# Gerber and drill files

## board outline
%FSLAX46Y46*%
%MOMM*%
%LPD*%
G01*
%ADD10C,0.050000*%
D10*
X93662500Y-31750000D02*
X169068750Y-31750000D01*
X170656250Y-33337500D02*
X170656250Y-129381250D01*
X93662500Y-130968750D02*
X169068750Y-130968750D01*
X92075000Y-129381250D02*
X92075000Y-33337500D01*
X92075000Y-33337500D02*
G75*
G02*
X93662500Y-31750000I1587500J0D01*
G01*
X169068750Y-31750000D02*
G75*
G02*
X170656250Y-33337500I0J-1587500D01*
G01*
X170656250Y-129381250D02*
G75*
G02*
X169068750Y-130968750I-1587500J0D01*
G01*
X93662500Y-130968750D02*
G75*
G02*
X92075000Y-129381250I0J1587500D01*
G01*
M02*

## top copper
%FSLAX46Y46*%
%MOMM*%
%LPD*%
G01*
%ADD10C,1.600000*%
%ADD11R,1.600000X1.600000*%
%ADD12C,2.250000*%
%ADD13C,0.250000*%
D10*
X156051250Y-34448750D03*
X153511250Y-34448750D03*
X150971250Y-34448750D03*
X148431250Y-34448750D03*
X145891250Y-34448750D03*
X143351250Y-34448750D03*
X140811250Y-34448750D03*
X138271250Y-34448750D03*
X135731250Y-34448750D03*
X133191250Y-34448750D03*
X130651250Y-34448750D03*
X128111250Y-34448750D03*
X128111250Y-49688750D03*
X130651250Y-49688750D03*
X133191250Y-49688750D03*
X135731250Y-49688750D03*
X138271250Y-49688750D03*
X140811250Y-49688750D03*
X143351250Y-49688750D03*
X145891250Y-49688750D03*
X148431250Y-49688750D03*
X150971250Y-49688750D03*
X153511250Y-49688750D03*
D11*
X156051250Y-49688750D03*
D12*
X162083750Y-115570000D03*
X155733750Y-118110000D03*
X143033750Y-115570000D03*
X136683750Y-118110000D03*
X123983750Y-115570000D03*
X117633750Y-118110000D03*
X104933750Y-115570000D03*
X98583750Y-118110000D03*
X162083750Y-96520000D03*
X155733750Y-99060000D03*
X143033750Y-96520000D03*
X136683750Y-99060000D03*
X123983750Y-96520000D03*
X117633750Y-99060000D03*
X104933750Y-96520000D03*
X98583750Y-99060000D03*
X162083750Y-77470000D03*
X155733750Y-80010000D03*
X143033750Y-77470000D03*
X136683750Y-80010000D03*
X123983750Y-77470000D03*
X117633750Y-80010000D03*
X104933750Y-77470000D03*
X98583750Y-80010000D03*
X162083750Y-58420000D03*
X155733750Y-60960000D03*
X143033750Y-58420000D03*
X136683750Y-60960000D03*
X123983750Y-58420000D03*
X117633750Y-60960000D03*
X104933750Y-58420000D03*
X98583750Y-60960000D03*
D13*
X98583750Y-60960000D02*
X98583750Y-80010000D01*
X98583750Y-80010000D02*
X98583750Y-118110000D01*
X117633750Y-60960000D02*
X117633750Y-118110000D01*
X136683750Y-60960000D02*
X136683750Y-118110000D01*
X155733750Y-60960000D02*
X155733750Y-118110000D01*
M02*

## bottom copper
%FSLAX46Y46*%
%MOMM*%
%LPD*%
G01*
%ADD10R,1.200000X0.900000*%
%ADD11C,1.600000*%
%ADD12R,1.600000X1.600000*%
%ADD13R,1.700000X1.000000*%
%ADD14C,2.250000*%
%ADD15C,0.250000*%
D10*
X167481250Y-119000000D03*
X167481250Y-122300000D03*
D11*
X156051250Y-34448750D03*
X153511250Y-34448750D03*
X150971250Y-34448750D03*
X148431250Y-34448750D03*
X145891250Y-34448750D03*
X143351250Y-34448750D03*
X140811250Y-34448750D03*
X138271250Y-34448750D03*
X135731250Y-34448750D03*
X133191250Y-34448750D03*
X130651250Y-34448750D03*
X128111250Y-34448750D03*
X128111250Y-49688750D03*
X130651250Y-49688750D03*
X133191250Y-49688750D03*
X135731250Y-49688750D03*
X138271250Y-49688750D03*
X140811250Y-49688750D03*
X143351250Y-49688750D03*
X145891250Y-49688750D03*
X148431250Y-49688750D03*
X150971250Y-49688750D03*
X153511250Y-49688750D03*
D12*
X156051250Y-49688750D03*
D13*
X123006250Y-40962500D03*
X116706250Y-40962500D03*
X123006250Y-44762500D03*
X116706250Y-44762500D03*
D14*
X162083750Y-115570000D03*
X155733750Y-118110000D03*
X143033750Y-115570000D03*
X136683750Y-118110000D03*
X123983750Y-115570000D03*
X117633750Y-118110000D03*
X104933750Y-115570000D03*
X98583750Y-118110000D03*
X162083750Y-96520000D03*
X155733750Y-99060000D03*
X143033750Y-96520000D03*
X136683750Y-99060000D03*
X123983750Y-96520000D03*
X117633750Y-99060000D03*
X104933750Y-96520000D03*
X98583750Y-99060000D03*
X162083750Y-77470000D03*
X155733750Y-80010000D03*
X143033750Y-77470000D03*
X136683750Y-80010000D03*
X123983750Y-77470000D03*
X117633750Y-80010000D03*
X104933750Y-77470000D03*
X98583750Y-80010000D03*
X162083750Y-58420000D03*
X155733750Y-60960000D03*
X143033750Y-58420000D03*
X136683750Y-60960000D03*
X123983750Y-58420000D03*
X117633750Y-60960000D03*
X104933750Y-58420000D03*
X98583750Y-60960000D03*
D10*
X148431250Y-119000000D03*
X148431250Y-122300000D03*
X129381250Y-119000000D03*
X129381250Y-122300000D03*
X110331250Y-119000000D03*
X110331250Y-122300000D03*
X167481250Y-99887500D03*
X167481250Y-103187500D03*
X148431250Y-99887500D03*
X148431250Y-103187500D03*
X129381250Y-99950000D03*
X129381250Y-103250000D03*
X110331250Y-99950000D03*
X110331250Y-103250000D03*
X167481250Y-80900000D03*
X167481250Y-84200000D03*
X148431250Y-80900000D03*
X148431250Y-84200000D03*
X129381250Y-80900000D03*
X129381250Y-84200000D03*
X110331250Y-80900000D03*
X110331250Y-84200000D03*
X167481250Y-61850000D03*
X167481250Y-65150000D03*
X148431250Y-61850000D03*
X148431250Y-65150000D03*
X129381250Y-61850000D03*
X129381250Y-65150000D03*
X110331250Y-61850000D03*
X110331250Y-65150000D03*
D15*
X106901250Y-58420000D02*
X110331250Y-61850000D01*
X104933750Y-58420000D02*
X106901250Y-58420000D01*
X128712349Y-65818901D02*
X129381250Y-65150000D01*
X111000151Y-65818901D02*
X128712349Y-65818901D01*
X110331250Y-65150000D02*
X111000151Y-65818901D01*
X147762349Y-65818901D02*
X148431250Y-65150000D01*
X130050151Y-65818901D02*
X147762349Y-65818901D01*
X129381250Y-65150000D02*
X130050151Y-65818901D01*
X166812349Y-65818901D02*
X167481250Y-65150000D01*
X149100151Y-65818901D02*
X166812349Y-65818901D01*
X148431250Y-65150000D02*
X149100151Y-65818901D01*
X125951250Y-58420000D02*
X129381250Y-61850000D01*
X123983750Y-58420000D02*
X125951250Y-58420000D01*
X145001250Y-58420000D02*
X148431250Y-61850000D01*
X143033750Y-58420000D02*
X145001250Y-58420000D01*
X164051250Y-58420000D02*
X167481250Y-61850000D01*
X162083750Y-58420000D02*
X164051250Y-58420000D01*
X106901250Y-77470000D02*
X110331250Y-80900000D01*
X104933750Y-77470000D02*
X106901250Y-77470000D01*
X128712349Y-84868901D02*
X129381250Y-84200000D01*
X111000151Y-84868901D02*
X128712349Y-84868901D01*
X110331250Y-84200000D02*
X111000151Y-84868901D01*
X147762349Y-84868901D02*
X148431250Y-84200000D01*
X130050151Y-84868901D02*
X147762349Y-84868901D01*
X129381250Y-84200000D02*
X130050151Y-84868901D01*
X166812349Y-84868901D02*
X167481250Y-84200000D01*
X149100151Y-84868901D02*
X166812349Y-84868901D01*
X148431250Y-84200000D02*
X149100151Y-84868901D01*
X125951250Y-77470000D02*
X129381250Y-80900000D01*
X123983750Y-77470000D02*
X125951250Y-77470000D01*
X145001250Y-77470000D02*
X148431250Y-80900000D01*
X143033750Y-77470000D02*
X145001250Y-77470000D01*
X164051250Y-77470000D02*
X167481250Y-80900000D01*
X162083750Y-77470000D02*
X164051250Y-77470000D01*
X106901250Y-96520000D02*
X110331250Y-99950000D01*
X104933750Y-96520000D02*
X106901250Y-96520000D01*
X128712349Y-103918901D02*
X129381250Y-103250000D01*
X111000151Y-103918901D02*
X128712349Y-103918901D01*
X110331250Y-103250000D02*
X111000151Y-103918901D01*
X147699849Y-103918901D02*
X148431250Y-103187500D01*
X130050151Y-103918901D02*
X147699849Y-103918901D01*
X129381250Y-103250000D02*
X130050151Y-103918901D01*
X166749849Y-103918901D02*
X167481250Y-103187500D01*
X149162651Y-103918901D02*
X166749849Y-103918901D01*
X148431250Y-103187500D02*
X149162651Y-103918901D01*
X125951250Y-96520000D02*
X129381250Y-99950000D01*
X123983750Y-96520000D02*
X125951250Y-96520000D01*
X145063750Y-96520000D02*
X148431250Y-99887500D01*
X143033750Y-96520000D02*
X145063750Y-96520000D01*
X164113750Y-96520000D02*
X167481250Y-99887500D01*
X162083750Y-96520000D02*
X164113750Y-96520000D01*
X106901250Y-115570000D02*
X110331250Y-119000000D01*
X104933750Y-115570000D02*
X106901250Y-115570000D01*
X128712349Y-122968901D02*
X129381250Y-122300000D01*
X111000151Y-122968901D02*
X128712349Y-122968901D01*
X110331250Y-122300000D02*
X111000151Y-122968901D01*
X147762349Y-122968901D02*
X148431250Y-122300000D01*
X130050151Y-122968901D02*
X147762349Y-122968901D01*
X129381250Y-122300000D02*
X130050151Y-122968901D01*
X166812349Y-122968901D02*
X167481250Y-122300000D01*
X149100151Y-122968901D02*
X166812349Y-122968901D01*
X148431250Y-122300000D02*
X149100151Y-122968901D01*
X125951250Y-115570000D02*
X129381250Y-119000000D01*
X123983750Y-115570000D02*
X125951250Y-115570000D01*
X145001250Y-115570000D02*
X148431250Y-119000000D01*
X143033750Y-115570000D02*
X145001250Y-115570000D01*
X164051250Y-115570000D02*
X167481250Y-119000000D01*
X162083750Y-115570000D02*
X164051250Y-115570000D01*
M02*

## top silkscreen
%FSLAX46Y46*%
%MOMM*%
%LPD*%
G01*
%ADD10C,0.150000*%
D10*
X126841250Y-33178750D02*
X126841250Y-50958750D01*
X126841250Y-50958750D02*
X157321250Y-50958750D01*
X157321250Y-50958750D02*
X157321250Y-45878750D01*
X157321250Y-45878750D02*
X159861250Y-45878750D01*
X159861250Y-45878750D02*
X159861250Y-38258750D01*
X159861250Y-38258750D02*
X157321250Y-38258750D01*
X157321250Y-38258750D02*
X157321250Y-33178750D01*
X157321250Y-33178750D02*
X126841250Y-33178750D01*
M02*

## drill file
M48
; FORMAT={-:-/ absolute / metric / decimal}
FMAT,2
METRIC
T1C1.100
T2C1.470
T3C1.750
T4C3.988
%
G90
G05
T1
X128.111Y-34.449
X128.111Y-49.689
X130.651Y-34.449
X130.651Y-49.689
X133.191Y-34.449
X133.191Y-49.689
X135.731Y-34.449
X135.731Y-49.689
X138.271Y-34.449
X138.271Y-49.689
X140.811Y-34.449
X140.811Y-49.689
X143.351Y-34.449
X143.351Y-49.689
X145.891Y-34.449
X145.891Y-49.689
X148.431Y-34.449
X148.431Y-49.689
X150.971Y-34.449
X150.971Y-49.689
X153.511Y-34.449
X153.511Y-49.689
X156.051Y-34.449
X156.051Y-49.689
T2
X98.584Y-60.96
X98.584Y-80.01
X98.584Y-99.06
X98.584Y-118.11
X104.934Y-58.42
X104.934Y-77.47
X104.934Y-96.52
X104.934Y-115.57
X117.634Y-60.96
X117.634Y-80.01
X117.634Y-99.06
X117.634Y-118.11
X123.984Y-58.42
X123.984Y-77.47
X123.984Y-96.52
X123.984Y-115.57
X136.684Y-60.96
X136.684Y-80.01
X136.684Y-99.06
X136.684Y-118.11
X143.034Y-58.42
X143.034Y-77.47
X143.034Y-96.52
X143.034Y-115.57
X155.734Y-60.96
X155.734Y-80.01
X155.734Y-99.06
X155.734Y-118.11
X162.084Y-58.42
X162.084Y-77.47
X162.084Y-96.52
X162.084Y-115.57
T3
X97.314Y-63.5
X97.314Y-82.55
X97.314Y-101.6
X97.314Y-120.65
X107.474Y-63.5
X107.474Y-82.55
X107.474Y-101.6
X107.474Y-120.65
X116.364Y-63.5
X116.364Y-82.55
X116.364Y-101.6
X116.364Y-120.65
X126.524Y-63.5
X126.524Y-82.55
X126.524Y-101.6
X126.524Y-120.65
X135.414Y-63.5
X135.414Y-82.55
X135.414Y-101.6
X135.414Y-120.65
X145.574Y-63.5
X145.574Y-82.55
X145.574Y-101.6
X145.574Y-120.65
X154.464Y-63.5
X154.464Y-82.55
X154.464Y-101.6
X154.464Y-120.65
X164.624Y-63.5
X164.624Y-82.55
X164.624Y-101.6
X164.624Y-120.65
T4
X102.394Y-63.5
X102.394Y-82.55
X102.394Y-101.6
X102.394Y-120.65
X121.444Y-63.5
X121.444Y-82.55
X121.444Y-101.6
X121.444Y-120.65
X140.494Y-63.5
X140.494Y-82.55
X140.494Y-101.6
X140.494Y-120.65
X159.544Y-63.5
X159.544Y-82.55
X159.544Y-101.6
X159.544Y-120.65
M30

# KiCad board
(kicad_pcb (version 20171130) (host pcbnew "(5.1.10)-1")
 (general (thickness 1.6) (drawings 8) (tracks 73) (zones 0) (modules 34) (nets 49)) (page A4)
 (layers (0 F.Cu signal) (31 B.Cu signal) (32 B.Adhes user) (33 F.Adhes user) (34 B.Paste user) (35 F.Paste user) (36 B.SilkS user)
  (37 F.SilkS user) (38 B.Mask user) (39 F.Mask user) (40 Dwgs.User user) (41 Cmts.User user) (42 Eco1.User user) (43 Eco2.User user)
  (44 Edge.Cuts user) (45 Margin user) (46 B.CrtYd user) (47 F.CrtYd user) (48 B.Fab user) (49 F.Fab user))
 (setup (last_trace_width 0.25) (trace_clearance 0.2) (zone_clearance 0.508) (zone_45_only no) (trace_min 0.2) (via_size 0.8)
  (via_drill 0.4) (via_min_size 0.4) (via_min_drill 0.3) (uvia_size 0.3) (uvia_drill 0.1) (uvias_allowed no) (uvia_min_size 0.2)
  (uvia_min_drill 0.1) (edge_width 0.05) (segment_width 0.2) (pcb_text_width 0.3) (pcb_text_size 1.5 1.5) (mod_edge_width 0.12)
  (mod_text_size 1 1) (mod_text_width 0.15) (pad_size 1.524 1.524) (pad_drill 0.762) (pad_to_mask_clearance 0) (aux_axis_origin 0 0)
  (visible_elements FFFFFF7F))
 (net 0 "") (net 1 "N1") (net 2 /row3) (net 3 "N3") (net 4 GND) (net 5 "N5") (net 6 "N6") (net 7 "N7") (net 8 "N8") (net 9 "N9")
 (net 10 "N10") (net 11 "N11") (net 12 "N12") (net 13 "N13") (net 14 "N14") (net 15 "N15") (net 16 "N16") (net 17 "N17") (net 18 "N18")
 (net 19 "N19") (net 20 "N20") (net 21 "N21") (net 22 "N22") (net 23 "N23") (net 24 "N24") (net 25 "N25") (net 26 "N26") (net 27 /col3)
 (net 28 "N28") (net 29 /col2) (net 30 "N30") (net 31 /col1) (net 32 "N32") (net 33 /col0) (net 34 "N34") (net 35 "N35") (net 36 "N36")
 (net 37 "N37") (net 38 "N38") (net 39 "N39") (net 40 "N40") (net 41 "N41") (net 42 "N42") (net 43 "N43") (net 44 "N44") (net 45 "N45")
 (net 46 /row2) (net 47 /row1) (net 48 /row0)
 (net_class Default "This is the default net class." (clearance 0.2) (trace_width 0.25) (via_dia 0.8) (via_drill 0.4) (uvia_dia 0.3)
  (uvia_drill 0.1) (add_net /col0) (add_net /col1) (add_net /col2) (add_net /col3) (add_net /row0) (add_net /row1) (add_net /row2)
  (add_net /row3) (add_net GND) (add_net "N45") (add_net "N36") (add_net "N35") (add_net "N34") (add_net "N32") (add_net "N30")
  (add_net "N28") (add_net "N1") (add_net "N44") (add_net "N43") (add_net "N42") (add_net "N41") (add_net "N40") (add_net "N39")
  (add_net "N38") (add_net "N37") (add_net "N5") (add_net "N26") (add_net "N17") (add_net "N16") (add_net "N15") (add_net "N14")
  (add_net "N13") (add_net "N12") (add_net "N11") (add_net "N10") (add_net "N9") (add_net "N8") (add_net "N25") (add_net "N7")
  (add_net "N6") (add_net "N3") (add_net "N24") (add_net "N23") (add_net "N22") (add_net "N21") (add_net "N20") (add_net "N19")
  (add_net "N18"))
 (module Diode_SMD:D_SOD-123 (layer B.Cu) (at 167.48125 120.65 90)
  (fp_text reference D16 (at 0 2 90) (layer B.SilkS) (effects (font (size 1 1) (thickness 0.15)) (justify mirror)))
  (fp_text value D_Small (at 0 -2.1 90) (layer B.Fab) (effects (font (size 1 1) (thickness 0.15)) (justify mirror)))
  (pad 2 smd rect (at 1.65 0 90) (size 0.9 1.2) (layers B.Cu B.Paste B.Mask) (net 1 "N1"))
  (pad 1 smd rect (at -1.65 0 90) (size 0.9 1.2) (layers B.Cu B.Paste B.Mask) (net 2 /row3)))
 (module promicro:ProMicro (layer B.Cu) (at 142.08125 42.06875 180)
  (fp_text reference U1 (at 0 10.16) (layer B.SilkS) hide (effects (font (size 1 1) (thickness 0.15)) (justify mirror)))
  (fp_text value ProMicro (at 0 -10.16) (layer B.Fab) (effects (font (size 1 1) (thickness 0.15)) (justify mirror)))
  (fp_line (start 15.24 8.89) (end 15.24 -8.89) (layer F.SilkS) (width 0.15))
  (fp_line (start 15.24 -8.89) (end -15.24 -8.89) (layer F.SilkS) (width 0.15))
  (fp_line (start -15.24 -8.89) (end -15.24 -3.81) (layer F.SilkS) (width 0.15))
  (fp_line (start -15.24 -3.81) (end -17.78 -3.81) (layer F.SilkS) (width 0.15))
  (fp_line (start -17.78 -3.81) (end -17.78 3.81) (layer F.SilkS) (width 0.15))
  (fp_line (start -17.78 3.81) (end -15.24 3.81) (layer F.SilkS) (width 0.15))
  (fp_line (start -15.24 3.81) (end -15.24 8.89) (layer F.SilkS) (width 0.15))
  (fp_line (start -15.24 8.89) (end 15.24 8.89) (layer F.SilkS) (width 0.15))
  (pad 24 thru_hole circle (at -13.97 7.62 180) (size 1.6 1.6) (drill 1.1) (layers *.Cu *.Mask B.SilkS) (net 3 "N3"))
  (pad 23 thru_hole circle (at -11.43 7.62 180) (size 1.6 1.6) (drill 1.1) (layers *.Cu *.Mask B.SilkS) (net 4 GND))
  (pad 22 thru_hole circle (at -8.89 7.62 180) (size 1.6 1.6) (drill 1.1) (layers *.Cu *.Mask B.SilkS) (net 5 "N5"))
  (pad 21 thru_hole circle (at -6.35 7.62 180) (size 1.6 1.6) (drill 1.1) (layers *.Cu *.Mask B.SilkS) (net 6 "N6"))
  (pad 20 thru_hole circle (at -3.81 7.62 180) (size 1.6 1.6) (drill 1.1) (layers *.Cu *.Mask B.SilkS) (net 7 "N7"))
  (pad 19 thru_hole circle (at -1.27 7.62 180) (size 1.6 1.6) (drill 1.1) (layers *.Cu *.Mask B.SilkS) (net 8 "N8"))
  (pad 18 thru_hole circle (at 1.27 7.62 180) (size 1.6 1.6) (drill 1.1) (layers *.Cu *.Mask B.SilkS) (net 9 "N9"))
  (pad 17 thru_hole circle (at 3.81 7.62 180) (size 1.6 1.6) (drill 1.1) (layers *.Cu *.Mask B.SilkS) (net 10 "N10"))
  (pad 16 thru_hole circle (at 6.35 7.62 180) (size 1.6 1.6) (drill 1.1) (layers *.Cu *.Mask B.SilkS) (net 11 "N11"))
  (pad 15 thru_hole circle (at 8.89 7.62 180) (size 1.6 1.6) (drill 1.1) (layers *.Cu *.Mask B.SilkS) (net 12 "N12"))
  (pad 14 thru_hole circle (at 11.43 7.62 180) (size 1.6 1.6) (drill 1.1) (layers *.Cu *.Mask B.SilkS) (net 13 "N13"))
  (pad 13 thru_hole circle (at 13.97 7.62 180) (size 1.6 1.6) (drill 1.1) (layers *.Cu *.Mask B.SilkS) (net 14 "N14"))
  (pad 12 thru_hole circle (at 13.97 -7.62 180) (size 1.6 1.6) (drill 1.1) (layers *.Cu *.Mask B.SilkS) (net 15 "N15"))
  (pad 11 thru_hole circle (at 11.43 -7.62 180) (size 1.6 1.6) (drill 1.1) (layers *.Cu *.Mask B.SilkS) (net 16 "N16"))
  (pad 10 thru_hole circle (at 8.89 -7.62 180) (size 1.6 1.6) (drill 1.1) (layers *.Cu *.Mask B.SilkS) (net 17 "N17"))
  (pad 9 thru_hole circle (at 6.35 -7.62 180) (size 1.6 1.6) (drill 1.1) (layers *.Cu *.Mask B.SilkS) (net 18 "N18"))
  (pad 8 thru_hole circle (at 3.81 -7.62 180) (size 1.6 1.6) (drill 1.1) (layers *.Cu *.Mask B.SilkS) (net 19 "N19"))
  (pad 7 thru_hole circle (at 1.27 -7.62 180) (size 1.6 1.6) (drill 1.1) (layers *.Cu *.Mask B.SilkS) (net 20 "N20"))
  (pad 6 thru_hole circle (at -1.27 -7.62 180) (size 1.6 1.6) (drill 1.1) (layers *.Cu *.Mask B.SilkS) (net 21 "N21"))
  (pad 5 thru_hole circle (at -3.81 -7.62 180) (size 1.6 1.6) (drill 1.1) (layers *.Cu *.Mask B.SilkS) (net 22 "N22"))
  (pad 4 thru_hole circle (at -6.35 -7.62 180) (size 1.6 1.6) (drill 1.1) (layers *.Cu *.Mask B.SilkS) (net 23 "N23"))
  (pad 3 thru_hole circle (at -8.89 -7.62 180) (size 1.6 1.6) (drill 1.1) (layers *.Cu *.Mask B.SilkS) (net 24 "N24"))
  (pad 2 thru_hole circle (at -11.43 -7.62 180) (size 1.6 1.6) (drill 1.1) (layers *.Cu *.Mask B.SilkS) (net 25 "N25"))
  (pad 1 thru_hole rect (at -13.97 -7.62 180) (size 1.6 1.6) (drill 1.1) (layers *.Cu *.Mask B.SilkS) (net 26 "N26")))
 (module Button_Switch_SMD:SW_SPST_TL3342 (layer B.Cu) (at 119.85625 42.8625)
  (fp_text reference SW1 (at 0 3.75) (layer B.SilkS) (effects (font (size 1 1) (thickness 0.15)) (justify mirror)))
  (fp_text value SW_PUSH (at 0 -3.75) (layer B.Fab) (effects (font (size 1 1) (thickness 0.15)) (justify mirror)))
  (pad 2 smd rect (at 3.15 -1.9) (size 1.7 1) (layers B.Cu B.Paste B.Mask) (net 4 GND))
  (pad 2 smd rect (at -3.15 -1.9) (size 1.7 1) (layers B.Cu B.Paste B.Mask) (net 4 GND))
  (pad 1 smd rect (at 3.15 1.9) (size 1.7 1) (layers B.Cu B.Paste B.Mask) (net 5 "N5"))
  (pad 1 smd rect (at -3.15 1.9) (size 1.7 1) (layers B.Cu B.Paste B.Mask) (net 5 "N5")))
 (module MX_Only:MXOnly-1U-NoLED (layer F.Cu) (at 159.54375 120.65)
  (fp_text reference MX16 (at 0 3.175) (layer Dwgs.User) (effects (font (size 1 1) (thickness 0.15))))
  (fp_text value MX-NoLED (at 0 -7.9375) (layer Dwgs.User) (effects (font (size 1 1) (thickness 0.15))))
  (pad 2 thru_hole circle (at 2.54 -5.08) (size 2.25 2.25) (drill 1.47) (layers *.Cu B.Mask) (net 1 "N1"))
  (pad "" np_thru_hole circle (at 0 0) (size 3.9878 3.9878) (drill 3.9878) (layers *.Cu *.Mask))
  (pad 1 thru_hole circle (at -3.81 -2.54) (size 2.25 2.25) (drill 1.47) (layers *.Cu B.Mask) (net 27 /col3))
  (pad "" np_thru_hole circle (at -5.08 0 48.0996) (size 1.75 1.75) (drill 1.75) (layers *.Cu *.Mask))
  (pad "" np_thru_hole circle (at 5.08 0 48.0996) (size 1.75 1.75) (drill 1.75) (layers *.Cu *.Mask)))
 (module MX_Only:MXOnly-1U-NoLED (layer F.Cu) (at 140.49375 120.65)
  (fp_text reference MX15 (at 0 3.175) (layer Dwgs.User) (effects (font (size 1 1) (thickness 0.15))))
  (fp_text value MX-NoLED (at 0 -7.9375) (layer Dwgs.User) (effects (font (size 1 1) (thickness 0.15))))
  (pad 2 thru_hole circle (at 2.54 -5.08) (size 2.25 2.25) (drill 1.47) (layers *.Cu B.Mask) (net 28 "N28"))
  (pad "" np_thru_hole circle (at 0 0) (size 3.9878 3.9878) (drill 3.9878) (layers *.Cu *.Mask))
  (pad 1 thru_hole circle (at -3.81 -2.54) (size 2.25 2.25) (drill 1.47) (layers *.Cu B.Mask) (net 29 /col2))
  (pad "" np_thru_hole circle (at -5.08 0 48.0996) (size 1.75 1.75) (drill 1.75) (layers *.Cu *.Mask))
  (pad "" np_thru_hole circle (at 5.08 0 48.0996) (size 1.75 1.75) (drill 1.75) (layers *.Cu *.Mask)))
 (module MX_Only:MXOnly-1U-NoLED (layer F.Cu) (at 121.44375 120.65)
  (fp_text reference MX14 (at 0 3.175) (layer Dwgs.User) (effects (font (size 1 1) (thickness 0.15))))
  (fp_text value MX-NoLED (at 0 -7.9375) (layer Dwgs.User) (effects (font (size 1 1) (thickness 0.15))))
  (pad 2 thru_hole circle (at 2.54 -5.08) (size 2.25 2.25) (drill 1.47) (layers *.Cu B.Mask) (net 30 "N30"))
  (pad "" np_thru_hole circle (at 0 0) (size 3.9878 3.9878) (drill 3.9878) (layers *.Cu *.Mask))
  (pad 1 thru_hole circle (at -3.81 -2.54) (size 2.25 2.25) (drill 1.47) (layers *.Cu B.Mask) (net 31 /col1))
  (pad "" np_thru_hole circle (at -5.08 0 48.0996) (size 1.75 1.75) (drill 1.75) (layers *.Cu *.Mask))
  (pad "" np_thru_hole circle (at 5.08 0 48.0996) (size 1.75 1.75) (drill 1.75) (layers *.Cu *.Mask)))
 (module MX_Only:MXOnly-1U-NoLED (layer F.Cu) (at 102.39375 120.65)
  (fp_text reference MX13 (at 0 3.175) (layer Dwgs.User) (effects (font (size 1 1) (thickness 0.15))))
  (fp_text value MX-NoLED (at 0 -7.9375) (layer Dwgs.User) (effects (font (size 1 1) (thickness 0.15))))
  (pad 2 thru_hole circle (at 2.54 -5.08) (size 2.25 2.25) (drill 1.47) (layers *.Cu B.Mask) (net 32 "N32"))
  (pad "" np_thru_hole circle (at 0 0) (size 3.9878 3.9878) (drill 3.9878) (layers *.Cu *.Mask))
  (pad 1 thru_hole circle (at -3.81 -2.54) (size 2.25 2.25) (drill 1.47) (layers *.Cu B.Mask) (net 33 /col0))
  (pad "" np_thru_hole circle (at -5.08 0 48.0996) (size 1.75 1.75) (drill 1.75) (layers *.Cu *.Mask))
  (pad "" np_thru_hole circle (at 5.08 0 48.0996) (size 1.75 1.75) (drill 1.75) (layers *.Cu *.Mask)))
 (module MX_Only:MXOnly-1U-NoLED (layer F.Cu) (at 159.54375 101.6)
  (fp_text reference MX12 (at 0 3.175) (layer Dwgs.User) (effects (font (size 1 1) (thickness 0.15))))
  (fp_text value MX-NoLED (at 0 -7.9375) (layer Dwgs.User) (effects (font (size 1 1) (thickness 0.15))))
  (pad 2 thru_hole circle (at 2.54 -5.08) (size 2.25 2.25) (drill 1.47) (layers *.Cu B.Mask) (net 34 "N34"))
  (pad "" np_thru_hole circle (at 0 0) (size 3.9878 3.9878) (drill 3.9878) (layers *.Cu *.Mask))
  (pad 1 thru_hole circle (at -3.81 -2.54) (size 2.25 2.25) (drill 1.47) (layers *.Cu B.Mask) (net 27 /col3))
  (pad "" np_thru_hole circle (at -5.08 0 48.0996) (size 1.75 1.75) (drill 1.75) (layers *.Cu *.Mask))
  (pad "" np_thru_hole circle (at 5.08 0 48.0996) (size 1.75 1.75) (drill 1.75) (layers *.Cu *.Mask)))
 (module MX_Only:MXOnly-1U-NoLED (layer F.Cu) (at 140.49375 101.6)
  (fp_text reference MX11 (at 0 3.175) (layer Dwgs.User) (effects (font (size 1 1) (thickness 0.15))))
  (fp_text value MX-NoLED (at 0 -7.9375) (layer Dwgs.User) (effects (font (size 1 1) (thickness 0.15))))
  (pad 2 thru_hole circle (at 2.54 -5.08) (size 2.25 2.25) (drill 1.47) (layers *.Cu B.Mask) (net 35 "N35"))
  (pad "" np_thru_hole circle (at 0 0) (size 3.9878 3.9878) (drill 3.9878) (layers *.Cu *.Mask))
  (pad 1 thru_hole circle (at -3.81 -2.54) (size 2.25 2.25) (drill 1.47) (layers *.Cu B.Mask) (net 29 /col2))
  (pad "" np_thru_hole circle (at -5.08 0 48.0996) (size 1.75 1.75) (drill 1.75) (layers *.Cu *.Mask))
  (pad "" np_thru_hole circle (at 5.08 0 48.0996) (size 1.75 1.75) (drill 1.75) (layers *.Cu *.Mask)))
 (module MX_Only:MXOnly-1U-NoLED (layer F.Cu) (at 121.44375 101.6)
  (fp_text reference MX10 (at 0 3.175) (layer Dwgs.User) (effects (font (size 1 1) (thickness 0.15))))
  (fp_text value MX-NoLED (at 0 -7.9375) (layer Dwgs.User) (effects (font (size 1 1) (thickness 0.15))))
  (pad 2 thru_hole circle (at 2.54 -5.08) (size 2.25 2.25) (drill 1.47) (layers *.Cu B.Mask) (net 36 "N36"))
  (pad "" np_thru_hole circle (at 0 0) (size 3.9878 3.9878) (drill 3.9878) (layers *.Cu *.Mask))
  (pad 1 thru_hole circle (at -3.81 -2.54) (size 2.25 2.25) (drill 1.47) (layers *.Cu B.Mask) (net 31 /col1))
  (pad "" np_thru_hole circle (at -5.08 0 48.0996) (size 1.75 1.75) (drill 1.75) (layers *.Cu *.Mask))
  (pad "" np_thru_hole circle (at 5.08 0 48.0996) (size 1.75 1.75) (drill 1.75) (layers *.Cu *.Mask)))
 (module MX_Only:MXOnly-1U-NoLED (layer F.Cu) (at 102.39375 101.6)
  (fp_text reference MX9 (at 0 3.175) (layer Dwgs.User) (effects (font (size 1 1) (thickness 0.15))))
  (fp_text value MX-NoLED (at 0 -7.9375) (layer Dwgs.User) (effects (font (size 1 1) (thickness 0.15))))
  (pad 2 thru_hole circle (at 2.54 -5.08) (size 2.25 2.25) (drill 1.47) (layers *.Cu B.Mask) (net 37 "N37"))
  (pad "" np_thru_hole circle (at 0 0) (size 3.9878 3.9878) (drill 3.9878) (layers *.Cu *.Mask))
  (pad 1 thru_hole circle (at -3.81 -2.54) (size 2.25 2.25) (drill 1.47) (layers *.Cu B.Mask) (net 33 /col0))
  (pad "" np_thru_hole circle (at -5.08 0 48.0996) (size 1.75 1.75) (drill 1.75) (layers *.Cu *.Mask))
  (pad "" np_thru_hole circle (at 5.08 0 48.0996) (size 1.75 1.75) (drill 1.75) (layers *.Cu *.Mask)))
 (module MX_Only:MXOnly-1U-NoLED (layer F.Cu) (at 159.54375 82.55)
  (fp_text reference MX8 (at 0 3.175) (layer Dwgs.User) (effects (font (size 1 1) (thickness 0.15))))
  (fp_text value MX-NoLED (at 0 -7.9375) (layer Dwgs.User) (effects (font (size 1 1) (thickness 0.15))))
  (pad 2 thru_hole circle (at 2.54 -5.08) (size 2.25 2.25) (drill 1.47) (layers *.Cu B.Mask) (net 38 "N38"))
  (pad "" np_thru_hole circle (at 0 0) (size 3.9878 3.9878) (drill 3.9878) (layers *.Cu *.Mask))
  (pad 1 thru_hole circle (at -3.81 -2.54) (size 2.25 2.25) (drill 1.47) (layers *.Cu B.Mask) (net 27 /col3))
  (pad "" np_thru_hole circle (at -5.08 0 48.0996) (size 1.75 1.75) (drill 1.75) (layers *.Cu *.Mask))
  (pad "" np_thru_hole circle (at 5.08 0 48.0996) (size 1.75 1.75) (drill 1.75) (layers *.Cu *.Mask)))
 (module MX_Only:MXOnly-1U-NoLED (layer F.Cu) (at 140.49375 82.55)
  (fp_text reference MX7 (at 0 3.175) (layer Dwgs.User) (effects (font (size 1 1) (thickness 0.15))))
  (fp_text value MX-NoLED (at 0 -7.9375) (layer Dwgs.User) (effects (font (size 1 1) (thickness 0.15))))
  (pad 2 thru_hole circle (at 2.54 -5.08) (size 2.25 2.25) (drill 1.47) (layers *.Cu B.Mask) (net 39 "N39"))
  (pad "" np_thru_hole circle (at 0 0) (size 3.9878 3.9878) (drill 3.9878) (layers *.Cu *.Mask))
  (pad 1 thru_hole circle (at -3.81 -2.54) (size 2.25 2.25) (drill 1.47) (layers *.Cu B.Mask) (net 29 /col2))
  (pad "" np_thru_hole circle (at -5.08 0 48.0996) (size 1.75 1.75) (drill 1.75) (layers *.Cu *.Mask))
  (pad "" np_thru_hole circle (at 5.08 0 48.0996) (size 1.75 1.75) (drill 1.75) (layers *.Cu *.Mask)))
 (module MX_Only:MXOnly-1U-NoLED (layer F.Cu) (at 121.44375 82.55)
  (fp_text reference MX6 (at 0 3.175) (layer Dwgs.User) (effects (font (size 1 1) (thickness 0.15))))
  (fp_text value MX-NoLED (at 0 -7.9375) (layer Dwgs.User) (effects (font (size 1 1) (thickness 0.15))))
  (pad 2 thru_hole circle (at 2.54 -5.08) (size 2.25 2.25) (drill 1.47) (layers *.Cu B.Mask) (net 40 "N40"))
  (pad "" np_thru_hole circle (at 0 0) (size 3.9878 3.9878) (drill 3.9878) (layers *.Cu *.Mask))
  (pad 1 thru_hole circle (at -3.81 -2.54) (size 2.25 2.25) (drill 1.47) (layers *.Cu B.Mask) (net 31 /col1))
  (pad "" np_thru_hole circle (at -5.08 0 48.0996) (size 1.75 1.75) (drill 1.75) (layers *.Cu *.Mask))
  (pad "" np_thru_hole circle (at 5.08 0 48.0996) (size 1.75 1.75) (drill 1.75) (layers *.Cu *.Mask)))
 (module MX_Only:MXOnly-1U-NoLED (layer F.Cu) (at 102.39375 82.55)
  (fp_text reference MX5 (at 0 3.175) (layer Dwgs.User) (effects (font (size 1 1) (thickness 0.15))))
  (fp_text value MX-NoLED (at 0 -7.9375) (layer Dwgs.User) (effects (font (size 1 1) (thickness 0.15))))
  (pad 2 thru_hole circle (at 2.54 -5.08) (size 2.25 2.25) (drill 1.47) (layers *.Cu B.Mask) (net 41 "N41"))
  (pad "" np_thru_hole circle (at 0 0) (size 3.9878 3.9878) (drill 3.9878) (layers *.Cu *.Mask))
  (pad 1 thru_hole circle (at -3.81 -2.54) (size 2.25 2.25) (drill 1.47) (layers *.Cu B.Mask) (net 33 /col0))
  (pad "" np_thru_hole circle (at -5.08 0 48.0996) (size 1.75 1.75) (drill 1.75) (layers *.Cu *.Mask))
  (pad "" np_thru_hole circle (at 5.08 0 48.0996) (size 1.75 1.75) (drill 1.75) (layers *.Cu *.Mask)))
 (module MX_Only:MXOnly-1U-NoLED (layer F.Cu) (at 159.54375 63.5)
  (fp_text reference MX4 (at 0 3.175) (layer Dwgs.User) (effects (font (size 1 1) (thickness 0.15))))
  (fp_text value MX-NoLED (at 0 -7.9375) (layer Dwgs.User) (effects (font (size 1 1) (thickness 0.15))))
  (pad 2 thru_hole circle (at 2.54 -5.08) (size 2.25 2.25) (drill 1.47) (layers *.Cu B.Mask) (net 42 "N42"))
  (pad "" np_thru_hole circle (at 0 0) (size 3.9878 3.9878) (drill 3.9878) (layers *.Cu *.Mask))
  (pad 1 thru_hole circle (at -3.81 -2.54) (size 2.25 2.25) (drill 1.47) (layers *.Cu B.Mask) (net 27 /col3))
  (pad "" np_thru_hole circle (at -5.08 0 48.0996) (size 1.75 1.75) (drill 1.75) (layers *.Cu *.Mask))
  (pad "" np_thru_hole circle (at 5.08 0 48.0996) (size 1.75 1.75) (drill 1.75) (layers *.Cu *.Mask)))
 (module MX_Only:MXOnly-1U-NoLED (layer F.Cu) (at 140.49375 63.5)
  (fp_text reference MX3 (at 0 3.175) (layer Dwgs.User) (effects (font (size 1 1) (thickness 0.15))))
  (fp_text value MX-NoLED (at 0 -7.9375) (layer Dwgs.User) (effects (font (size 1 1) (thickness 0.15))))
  (pad 2 thru_hole circle (at 2.54 -5.08) (size 2.25 2.25) (drill 1.47) (layers *.Cu B.Mask) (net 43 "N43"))
  (pad "" np_thru_hole circle (at 0 0) (size 3.9878 3.9878) (drill 3.9878) (layers *.Cu *.Mask))
  (pad 1 thru_hole circle (at -3.81 -2.54) (size 2.25 2.25) (drill 1.47) (layers *.Cu B.Mask) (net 29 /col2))
  (pad "" np_thru_hole circle (at -5.08 0 48.0996) (size 1.75 1.75) (drill 1.75) (layers *.Cu *.Mask))
  (pad "" np_thru_hole circle (at 5.08 0 48.0996) (size 1.75 1.75) (drill 1.75) (layers *.Cu *.Mask)))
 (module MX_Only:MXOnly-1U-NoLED (layer F.Cu) (at 121.44375 63.5)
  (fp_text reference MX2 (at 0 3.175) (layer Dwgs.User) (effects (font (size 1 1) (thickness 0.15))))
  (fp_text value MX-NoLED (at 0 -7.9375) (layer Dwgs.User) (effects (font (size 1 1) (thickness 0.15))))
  (pad 2 thru_hole circle (at 2.54 -5.08) (size 2.25 2.25) (drill 1.47) (layers *.Cu B.Mask) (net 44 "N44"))
  (pad "" np_thru_hole circle (at 0 0) (size 3.9878 3.9878) (drill 3.9878) (layers *.Cu *.Mask))
  (pad 1 thru_hole circle (at -3.81 -2.54) (size 2.25 2.25) (drill 1.47) (layers *.Cu B.Mask) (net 31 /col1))
  (pad "" np_thru_hole circle (at -5.08 0 48.0996) (size 1.75 1.75) (drill 1.75) (layers *.Cu *.Mask))
  (pad "" np_thru_hole circle (at 5.08 0 48.0996) (size 1.75 1.75) (drill 1.75) (layers *.Cu *.Mask)))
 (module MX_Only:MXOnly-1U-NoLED (layer F.Cu) (at 102.39375 63.5)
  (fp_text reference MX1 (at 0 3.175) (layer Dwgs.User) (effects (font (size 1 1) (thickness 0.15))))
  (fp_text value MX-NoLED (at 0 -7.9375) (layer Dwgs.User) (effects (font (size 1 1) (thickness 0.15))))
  (pad 2 thru_hole circle (at 2.54 -5.08) (size 2.25 2.25) (drill 1.47) (layers *.Cu B.Mask) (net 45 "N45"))
  (pad "" np_thru_hole circle (at 0 0) (size 3.9878 3.9878) (drill 3.9878) (layers *.Cu *.Mask))
  (pad 1 thru_hole circle (at -3.81 -2.54) (size 2.25 2.25) (drill 1.47) (layers *.Cu B.Mask) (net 33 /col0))
  (pad "" np_thru_hole circle (at -5.08 0 48.0996) (size 1.75 1.75) (drill 1.75) (layers *.Cu *.Mask))
  (pad "" np_thru_hole circle (at 5.08 0 48.0996) (size 1.75 1.75) (drill 1.75) (layers *.Cu *.Mask)))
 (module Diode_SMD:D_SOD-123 (layer B.Cu) (at 148.43125 120.65 90)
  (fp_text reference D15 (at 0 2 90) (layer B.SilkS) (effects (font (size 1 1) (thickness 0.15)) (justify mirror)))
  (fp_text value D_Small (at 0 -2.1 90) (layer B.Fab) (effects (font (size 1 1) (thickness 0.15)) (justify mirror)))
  (pad 2 smd rect (at 1.65 0 90) (size 0.9 1.2) (layers B.Cu B.Paste B.Mask) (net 28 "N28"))
  (pad 1 smd rect (at -1.65 0 90) (size 0.9 1.2) (layers B.Cu B.Paste B.Mask) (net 2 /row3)))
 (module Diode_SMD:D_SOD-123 (layer B.Cu) (at 129.38125 120.65 90)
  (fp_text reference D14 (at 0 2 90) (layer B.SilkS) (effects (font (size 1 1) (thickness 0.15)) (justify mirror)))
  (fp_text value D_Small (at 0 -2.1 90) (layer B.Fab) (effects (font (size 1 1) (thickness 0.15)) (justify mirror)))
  (pad 2 smd rect (at 1.65 0 90) (size 0.9 1.2) (layers B.Cu B.Paste B.Mask) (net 30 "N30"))
  (pad 1 smd rect (at -1.65 0 90) (size 0.9 1.2) (layers B.Cu B.Paste B.Mask) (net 2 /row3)))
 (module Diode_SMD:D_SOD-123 (layer B.Cu) (at 110.33125 120.65 90)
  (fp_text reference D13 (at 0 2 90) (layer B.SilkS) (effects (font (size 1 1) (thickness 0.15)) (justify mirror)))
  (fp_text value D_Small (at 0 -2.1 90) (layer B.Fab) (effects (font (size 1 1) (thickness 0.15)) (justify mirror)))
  (pad 2 smd rect (at 1.65 0 90) (size 0.9 1.2) (layers B.Cu B.Paste B.Mask) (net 32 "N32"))
  (pad 1 smd rect (at -1.65 0 90) (size 0.9 1.2) (layers B.Cu B.Paste B.Mask) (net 2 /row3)))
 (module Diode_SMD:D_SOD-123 (layer B.Cu) (at 167.48125 101.5375 90)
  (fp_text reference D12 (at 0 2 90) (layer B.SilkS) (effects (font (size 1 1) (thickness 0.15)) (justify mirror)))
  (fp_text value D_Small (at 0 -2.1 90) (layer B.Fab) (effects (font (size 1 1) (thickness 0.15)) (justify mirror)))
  (pad 2 smd rect (at 1.65 0 90) (size 0.9 1.2) (layers B.Cu B.Paste B.Mask) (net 34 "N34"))
  (pad 1 smd rect (at -1.65 0 90) (size 0.9 1.2) (layers B.Cu B.Paste B.Mask) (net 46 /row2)))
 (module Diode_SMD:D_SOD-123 (layer B.Cu) (at 148.43125 101.5375 90)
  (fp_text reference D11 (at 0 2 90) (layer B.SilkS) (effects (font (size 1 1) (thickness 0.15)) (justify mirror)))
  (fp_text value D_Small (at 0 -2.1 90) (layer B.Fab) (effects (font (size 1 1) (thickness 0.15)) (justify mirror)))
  (pad 2 smd rect (at 1.65 0 90) (size 0.9 1.2) (layers B.Cu B.Paste B.Mask) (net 35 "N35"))
  (pad 1 smd rect (at -1.65 0 90) (size 0.9 1.2) (layers B.Cu B.Paste B.Mask) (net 46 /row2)))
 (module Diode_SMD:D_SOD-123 (layer B.Cu) (at 129.38125 101.6 90)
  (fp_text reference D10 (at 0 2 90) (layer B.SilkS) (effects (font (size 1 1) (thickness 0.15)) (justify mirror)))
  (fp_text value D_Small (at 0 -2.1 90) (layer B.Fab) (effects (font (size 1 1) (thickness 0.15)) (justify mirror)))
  (pad 2 smd rect (at 1.65 0 90) (size 0.9 1.2) (layers B.Cu B.Paste B.Mask) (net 36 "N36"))
  (pad 1 smd rect (at -1.65 0 90) (size 0.9 1.2) (layers B.Cu B.Paste B.Mask) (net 46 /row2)))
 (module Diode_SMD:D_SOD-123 (layer B.Cu) (at 110.33125 101.6 90)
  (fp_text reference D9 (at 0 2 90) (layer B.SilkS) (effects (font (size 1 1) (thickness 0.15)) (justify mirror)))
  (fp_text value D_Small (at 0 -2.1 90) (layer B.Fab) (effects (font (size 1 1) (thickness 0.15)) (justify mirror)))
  (pad 2 smd rect (at 1.65 0 90) (size 0.9 1.2) (layers B.Cu B.Paste B.Mask) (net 37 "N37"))
  (pad 1 smd rect (at -1.65 0 90) (size 0.9 1.2) (layers B.Cu B.Paste B.Mask) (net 46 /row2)))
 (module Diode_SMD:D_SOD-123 (layer B.Cu) (at 167.48125 82.55 90)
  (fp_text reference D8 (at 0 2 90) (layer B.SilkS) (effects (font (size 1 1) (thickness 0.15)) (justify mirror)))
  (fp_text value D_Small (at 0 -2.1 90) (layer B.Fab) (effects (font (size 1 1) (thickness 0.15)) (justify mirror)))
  (pad 2 smd rect (at 1.65 0 90) (size 0.9 1.2) (layers B.Cu B.Paste B.Mask) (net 38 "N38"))
  (pad 1 smd rect (at -1.65 0 90) (size 0.9 1.2) (layers B.Cu B.Paste B.Mask) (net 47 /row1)))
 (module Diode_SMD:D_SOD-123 (layer B.Cu) (at 148.43125 82.55 90)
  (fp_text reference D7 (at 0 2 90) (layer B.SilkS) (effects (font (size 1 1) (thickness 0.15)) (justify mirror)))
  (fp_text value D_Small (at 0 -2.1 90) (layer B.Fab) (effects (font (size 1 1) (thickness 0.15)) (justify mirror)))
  (pad 2 smd rect (at 1.65 0 90) (size 0.9 1.2) (layers B.Cu B.Paste B.Mask) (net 39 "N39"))
  (pad 1 smd rect (at -1.65 0 90) (size 0.9 1.2) (layers B.Cu B.Paste B.Mask) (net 47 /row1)))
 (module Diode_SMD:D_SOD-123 (layer B.Cu) (at 129.38125 82.55 90)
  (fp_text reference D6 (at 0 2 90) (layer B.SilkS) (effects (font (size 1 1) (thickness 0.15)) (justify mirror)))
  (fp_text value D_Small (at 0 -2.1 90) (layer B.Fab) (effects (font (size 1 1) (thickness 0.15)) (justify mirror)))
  (pad 2 smd rect (at 1.65 0 90) (size 0.9 1.2) (layers B.Cu B.Paste B.Mask) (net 40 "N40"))
  (pad 1 smd rect (at -1.65 0 90) (size 0.9 1.2) (layers B.Cu B.Paste B.Mask) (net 47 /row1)))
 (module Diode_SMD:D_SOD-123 (layer B.Cu) (at 110.33125 82.55 90)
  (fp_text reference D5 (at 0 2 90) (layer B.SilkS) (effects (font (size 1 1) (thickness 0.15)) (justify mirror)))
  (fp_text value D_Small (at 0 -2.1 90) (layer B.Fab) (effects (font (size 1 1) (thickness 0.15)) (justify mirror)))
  (pad 2 smd rect (at 1.65 0 90) (size 0.9 1.2) (layers B.Cu B.Paste B.Mask) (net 41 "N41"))
  (pad 1 smd rect (at -1.65 0 90) (size 0.9 1.2) (layers B.Cu B.Paste B.Mask) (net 47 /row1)))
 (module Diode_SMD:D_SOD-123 (layer B.Cu) (at 167.48125 63.5 90)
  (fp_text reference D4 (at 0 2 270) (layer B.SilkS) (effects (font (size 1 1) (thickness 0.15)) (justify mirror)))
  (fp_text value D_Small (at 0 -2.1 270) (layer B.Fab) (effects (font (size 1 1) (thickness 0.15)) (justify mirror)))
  (pad 2 smd rect (at 1.65 0 90) (size 0.9 1.2) (layers B.Cu B.Paste B.Mask) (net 42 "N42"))
  (pad 1 smd rect (at -1.65 0 90) (size 0.9 1.2) (layers B.Cu B.Paste B.Mask) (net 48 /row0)))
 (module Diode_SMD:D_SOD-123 (layer B.Cu) (at 148.43125 63.5 90)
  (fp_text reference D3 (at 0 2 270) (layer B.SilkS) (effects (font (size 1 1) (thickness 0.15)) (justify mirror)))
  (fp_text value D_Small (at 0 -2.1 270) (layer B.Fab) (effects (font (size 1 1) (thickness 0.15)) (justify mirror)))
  (pad 2 smd rect (at 1.65 0 90) (size 0.9 1.2) (layers B.Cu B.Paste B.Mask) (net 43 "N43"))
  (pad 1 smd rect (at -1.65 0 90) (size 0.9 1.2) (layers B.Cu B.Paste B.Mask) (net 48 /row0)))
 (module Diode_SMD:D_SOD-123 (layer B.Cu) (at 129.38125 63.5 90)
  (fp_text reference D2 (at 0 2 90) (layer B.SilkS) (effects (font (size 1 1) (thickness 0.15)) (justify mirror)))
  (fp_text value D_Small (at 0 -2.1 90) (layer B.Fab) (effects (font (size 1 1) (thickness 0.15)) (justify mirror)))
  (pad 2 smd rect (at 1.65 0 90) (size 0.9 1.2) (layers B.Cu B.Paste B.Mask) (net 44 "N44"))
  (pad 1 smd rect (at -1.65 0 90) (size 0.9 1.2) (layers B.Cu B.Paste B.Mask) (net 48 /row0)))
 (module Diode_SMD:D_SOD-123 (layer B.Cu) (at 110.33125 63.5 90)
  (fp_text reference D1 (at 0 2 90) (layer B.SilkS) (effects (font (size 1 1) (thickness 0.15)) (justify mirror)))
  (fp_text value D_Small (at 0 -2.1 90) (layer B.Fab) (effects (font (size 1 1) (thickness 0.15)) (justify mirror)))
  (pad 2 smd rect (at 1.65 0 90) (size 0.9 1.2) (layers B.Cu B.Paste B.Mask) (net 45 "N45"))
  (pad 1 smd rect (at -1.65 0 90) (size 0.9 1.2) (layers B.Cu B.Paste B.Mask) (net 48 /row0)))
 (gr_line (start 93.6625 31.75) (end 169.06875 31.75) (layer Edge.Cuts) (width 0.05))
 (gr_line (start 170.65625 33.3375) (end 170.65625 129.38125) (layer Edge.Cuts) (width 0.05))
 (gr_line (start 93.6625 130.96875) (end 169.06875 130.96875) (layer Edge.Cuts) (width 0.05))
 (gr_line (start 92.075 129.38125) (end 92.075 33.3375) (layer Edge.Cuts) (width 0.05))
 (gr_arc (start 93.6625 33.3375) (end 93.6625 31.75) (angle -90) (layer Edge.Cuts) (width 0.05))
 (gr_arc (start 169.06875 33.3375) (end 170.65625 33.3375) (angle -90) (layer Edge.Cuts) (width 0.05))
 (gr_arc (start 169.06875 129.38125) (end 169.06875 130.96875) (angle -90) (layer Edge.Cuts) (width 0.05))
 (gr_arc (start 93.6625 129.38125) (end 92.075 129.38125) (angle -90) (layer Edge.Cuts) (width 0.05))
 (segment (start 106.90125 58.42) (end 110.33125 61.85) (width 0.25) (layer B.Cu) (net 45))
 (segment (start 104.93375 58.42) (end 106.90125 58.42) (width 0.25) (layer B.Cu) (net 45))
 (segment (start 128.712349 65.818901) (end 129.38125 65.15) (width 0.25) (layer B.Cu) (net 48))
 (segment (start 111.000151 65.818901) (end 128.712349 65.818901) (width 0.25) (layer B.Cu) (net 48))
 (segment (start 110.33125 65.15) (end 111.000151 65.818901) (width 0.25) (layer B.Cu) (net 48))
 (segment (start 147.762349 65.818901) (end 148.43125 65.15) (width 0.25) (layer B.Cu) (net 48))
 (segment (start 130.050151 65.818901) (end 147.762349 65.818901) (width 0.25) (layer B.Cu) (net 48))
 (segment (start 129.38125 65.15) (end 130.050151 65.818901) (width 0.25) (layer B.Cu) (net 48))
 (segment (start 166.812349 65.818901) (end 167.48125 65.15) (width 0.25) (layer B.Cu) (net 48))
 (segment (start 149.100151 65.818901) (end 166.812349 65.818901) (width 0.25) (layer B.Cu) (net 48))
 (segment (start 148.43125 65.15) (end 149.100151 65.818901) (width 0.25) (layer B.Cu) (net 48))
 (segment (start 125.95125 58.42) (end 129.38125 61.85) (width 0.25) (layer B.Cu) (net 44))
 (segment (start 123.98375 58.42) (end 125.95125 58.42) (width 0.25) (layer B.Cu) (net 44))
 (segment (start 145.00125 58.42) (end 148.43125 61.85) (width 0.25) (layer B.Cu) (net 43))
 (segment (start 143.03375 58.42) (end 145.00125 58.42) (width 0.25) (layer B.Cu) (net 43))
 (segment (start 164.05125 58.42) (end 167.48125 61.85) (width 0.25) (layer B.Cu) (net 42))
 (segment (start 162.08375 58.42) (end 164.05125 58.42) (width 0.25) (layer B.Cu) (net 42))
 (segment (start 106.90125 77.47) (end 110.33125 80.9) (width 0.25) (layer B.Cu) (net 41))
 (segment (start 104.93375 77.47) (end 106.90125 77.47) (width 0.25) (layer B.Cu) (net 41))
 (segment (start 128.712349 84.868901) (end 129.38125 84.2) (width 0.25) (layer B.Cu) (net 47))
 (segment (start 111.000151 84.868901) (end 128.712349 84.868901) (width 0.25) (layer B.Cu) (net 47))
 (segment (start 110.33125 84.2) (end 111.000151 84.868901) (width 0.25) (layer B.Cu) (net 47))
 (segment (start 147.762349 84.868901) (end 148.43125 84.2) (width 0.25) (layer B.Cu) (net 47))
 (segment (start 130.050151 84.868901) (end 147.762349 84.868901) (width 0.25) (layer B.Cu) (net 47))
 (segment (start 129.38125 84.2) (end 130.050151 84.868901) (width 0.25) (layer B.Cu) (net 47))
 (segment (start 166.812349 84.868901) (end 167.48125 84.2) (width 0.25) (layer B.Cu) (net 47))
 (segment (start 149.100151 84.868901) (end 166.812349 84.868901) (width 0.25) (layer B.Cu) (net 47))
 (segment (start 148.43125 84.2) (end 149.100151 84.868901) (width 0.25) (layer B.Cu) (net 47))
 (segment (start 125.95125 77.47) (end 129.38125 80.9) (width 0.25) (layer B.Cu) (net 40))
 (segment (start 123.98375 77.47) (end 125.95125 77.47) (width 0.25) (layer B.Cu) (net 40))
 (segment (start 145.00125 77.47) (end 148.43125 80.9) (width 0.25) (layer B.Cu) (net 39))
 (segment (start 143.03375 77.47) (end 145.00125 77.47) (width 0.25) (layer B.Cu) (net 39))
 (segment (start 164.05125 77.47) (end 167.48125 80.9) (width 0.25) (layer B.Cu) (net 38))
 (segment (start 162.08375 77.47) (end 164.05125 77.47) (width 0.25) (layer B.Cu) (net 38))
 (segment (start 106.90125 96.52) (end 110.33125 99.95) (width 0.25) (layer B.Cu) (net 37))
 (segment (start 104.93375 96.52) (end 106.90125 96.52) (width 0.25) (layer B.Cu) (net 37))
 (segment (start 128.712349 103.918901) (end 129.38125 103.25) (width 0.25) (layer B.Cu) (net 46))
 (segment (start 111.000151 103.918901) (end 128.712349 103.918901) (width 0.25) (layer B.Cu) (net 46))
 (segment (start 110.33125 103.25) (end 111.000151 103.918901) (width 0.25) (layer B.Cu) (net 46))
 (segment (start 147.699849 103.918901) (end 148.43125 103.1875) (width 0.25) (layer B.Cu) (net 46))
 (segment (start 130.050151 103.918901) (end 147.699849 103.918901) (width 0.25) (layer B.Cu) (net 46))
 (segment (start 129.38125 103.25) (end 130.050151 103.918901) (width 0.25) (layer B.Cu) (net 46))
 (segment (start 166.749849 103.918901) (end 167.48125 103.1875) (width 0.25) (layer B.Cu) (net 46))
 (segment (start 149.162651 103.918901) (end 166.749849 103.918901) (width 0.25) (layer B.Cu) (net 46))
 (segment (start 148.43125 103.1875) (end 149.162651 103.918901) (width 0.25) (layer B.Cu) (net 46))
 (segment (start 125.95125 96.52) (end 129.38125 99.95) (width 0.25) (layer B.Cu) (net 36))
 (segment (start 123.98375 96.52) (end 125.95125 96.52) (width 0.25) (layer B.Cu) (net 36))
 (segment (start 145.06375 96.52) (end 148.43125 99.8875) (width 0.25) (layer B.Cu) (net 35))
 (segment (start 143.03375 96.52) (end 145.06375 96.52) (width 0.25) (layer B.Cu) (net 35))
 (segment (start 164.11375 96.52) (end 167.48125 99.8875) (width 0.25) (layer B.Cu) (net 34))
 (segment (start 162.08375 96.52) (end 164.11375 96.52) (width 0.25) (layer B.Cu) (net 34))
 (segment (start 106.90125 115.57) (end 110.33125 119) (width 0.25) (layer B.Cu) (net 32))
 (segment (start 104.93375 115.57) (end 106.90125 115.57) (width 0.25) (layer B.Cu) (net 32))
 (segment (start 128.712349 122.968901) (end 129.38125 122.3) (width 0.25) (layer B.Cu) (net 2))
 (segment (start 111.000151 122.968901) (end 128.712349 122.968901) (width 0.25) (layer B.Cu) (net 2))
 (segment (start 110.33125 122.3) (end 111.000151 122.968901) (width 0.25) (layer B.Cu) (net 2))
 (segment (start 147.762349 122.968901) (end 148.43125 122.3) (width 0.25) (layer B.Cu) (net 2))
 (segment (start 130.050151 122.968901) (end 147.762349 122.968901) (width 0.25) (layer B.Cu) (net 2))
 (segment (start 129.38125 122.3) (end 130.050151 122.968901) (width 0.25) (layer B.Cu) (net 2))
 (segment (start 166.812349 122.968901) (end 167.48125 122.3) (width 0.25) (layer B.Cu) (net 2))
 (segment (start 149.100151 122.968901) (end 166.812349 122.968901) (width 0.25) (layer B.Cu) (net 2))
 (segment (start 148.43125 122.3) (end 149.100151 122.968901) (width 0.25) (layer B.Cu) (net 2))
 (segment (start 125.95125 115.57) (end 129.38125 119) (width 0.25) (layer B.Cu) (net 30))
 (segment (start 123.98375 115.57) (end 125.95125 115.57) (width 0.25) (layer B.Cu) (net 30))
 (segment (start 145.00125 115.57) (end 148.43125 119) (width 0.25) (layer B.Cu) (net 28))
 (segment (start 143.03375 115.57) (end 145.00125 115.57) (width 0.25) (layer B.Cu) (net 28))
 (segment (start 164.05125 115.57) (end 167.48125 119) (width 0.25) (layer B.Cu) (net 1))
 (segment (start 162.08375 115.57) (end 164.05125 115.57) (width 0.25) (layer B.Cu) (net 1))
 (segment (start 98.58375 60.96) (end 98.58375 80.01) (width 0.25) (layer F.Cu) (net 33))
 (segment (start 98.58375 80.01) (end 98.58375 118.11) (width 0.25) (layer F.Cu) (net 33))
 (segment (start 117.63375 60.96) (end 117.63375 118.11) (width 0.25) (layer F.Cu) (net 31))
 (segment (start 136.68375 60.96) (end 136.68375 118.11) (width 0.25) (layer F.Cu) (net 29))
 (segment (start 155.73375 60.96) (end 155.73375 118.11) (width 0.25) (layer F.Cu) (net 27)))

